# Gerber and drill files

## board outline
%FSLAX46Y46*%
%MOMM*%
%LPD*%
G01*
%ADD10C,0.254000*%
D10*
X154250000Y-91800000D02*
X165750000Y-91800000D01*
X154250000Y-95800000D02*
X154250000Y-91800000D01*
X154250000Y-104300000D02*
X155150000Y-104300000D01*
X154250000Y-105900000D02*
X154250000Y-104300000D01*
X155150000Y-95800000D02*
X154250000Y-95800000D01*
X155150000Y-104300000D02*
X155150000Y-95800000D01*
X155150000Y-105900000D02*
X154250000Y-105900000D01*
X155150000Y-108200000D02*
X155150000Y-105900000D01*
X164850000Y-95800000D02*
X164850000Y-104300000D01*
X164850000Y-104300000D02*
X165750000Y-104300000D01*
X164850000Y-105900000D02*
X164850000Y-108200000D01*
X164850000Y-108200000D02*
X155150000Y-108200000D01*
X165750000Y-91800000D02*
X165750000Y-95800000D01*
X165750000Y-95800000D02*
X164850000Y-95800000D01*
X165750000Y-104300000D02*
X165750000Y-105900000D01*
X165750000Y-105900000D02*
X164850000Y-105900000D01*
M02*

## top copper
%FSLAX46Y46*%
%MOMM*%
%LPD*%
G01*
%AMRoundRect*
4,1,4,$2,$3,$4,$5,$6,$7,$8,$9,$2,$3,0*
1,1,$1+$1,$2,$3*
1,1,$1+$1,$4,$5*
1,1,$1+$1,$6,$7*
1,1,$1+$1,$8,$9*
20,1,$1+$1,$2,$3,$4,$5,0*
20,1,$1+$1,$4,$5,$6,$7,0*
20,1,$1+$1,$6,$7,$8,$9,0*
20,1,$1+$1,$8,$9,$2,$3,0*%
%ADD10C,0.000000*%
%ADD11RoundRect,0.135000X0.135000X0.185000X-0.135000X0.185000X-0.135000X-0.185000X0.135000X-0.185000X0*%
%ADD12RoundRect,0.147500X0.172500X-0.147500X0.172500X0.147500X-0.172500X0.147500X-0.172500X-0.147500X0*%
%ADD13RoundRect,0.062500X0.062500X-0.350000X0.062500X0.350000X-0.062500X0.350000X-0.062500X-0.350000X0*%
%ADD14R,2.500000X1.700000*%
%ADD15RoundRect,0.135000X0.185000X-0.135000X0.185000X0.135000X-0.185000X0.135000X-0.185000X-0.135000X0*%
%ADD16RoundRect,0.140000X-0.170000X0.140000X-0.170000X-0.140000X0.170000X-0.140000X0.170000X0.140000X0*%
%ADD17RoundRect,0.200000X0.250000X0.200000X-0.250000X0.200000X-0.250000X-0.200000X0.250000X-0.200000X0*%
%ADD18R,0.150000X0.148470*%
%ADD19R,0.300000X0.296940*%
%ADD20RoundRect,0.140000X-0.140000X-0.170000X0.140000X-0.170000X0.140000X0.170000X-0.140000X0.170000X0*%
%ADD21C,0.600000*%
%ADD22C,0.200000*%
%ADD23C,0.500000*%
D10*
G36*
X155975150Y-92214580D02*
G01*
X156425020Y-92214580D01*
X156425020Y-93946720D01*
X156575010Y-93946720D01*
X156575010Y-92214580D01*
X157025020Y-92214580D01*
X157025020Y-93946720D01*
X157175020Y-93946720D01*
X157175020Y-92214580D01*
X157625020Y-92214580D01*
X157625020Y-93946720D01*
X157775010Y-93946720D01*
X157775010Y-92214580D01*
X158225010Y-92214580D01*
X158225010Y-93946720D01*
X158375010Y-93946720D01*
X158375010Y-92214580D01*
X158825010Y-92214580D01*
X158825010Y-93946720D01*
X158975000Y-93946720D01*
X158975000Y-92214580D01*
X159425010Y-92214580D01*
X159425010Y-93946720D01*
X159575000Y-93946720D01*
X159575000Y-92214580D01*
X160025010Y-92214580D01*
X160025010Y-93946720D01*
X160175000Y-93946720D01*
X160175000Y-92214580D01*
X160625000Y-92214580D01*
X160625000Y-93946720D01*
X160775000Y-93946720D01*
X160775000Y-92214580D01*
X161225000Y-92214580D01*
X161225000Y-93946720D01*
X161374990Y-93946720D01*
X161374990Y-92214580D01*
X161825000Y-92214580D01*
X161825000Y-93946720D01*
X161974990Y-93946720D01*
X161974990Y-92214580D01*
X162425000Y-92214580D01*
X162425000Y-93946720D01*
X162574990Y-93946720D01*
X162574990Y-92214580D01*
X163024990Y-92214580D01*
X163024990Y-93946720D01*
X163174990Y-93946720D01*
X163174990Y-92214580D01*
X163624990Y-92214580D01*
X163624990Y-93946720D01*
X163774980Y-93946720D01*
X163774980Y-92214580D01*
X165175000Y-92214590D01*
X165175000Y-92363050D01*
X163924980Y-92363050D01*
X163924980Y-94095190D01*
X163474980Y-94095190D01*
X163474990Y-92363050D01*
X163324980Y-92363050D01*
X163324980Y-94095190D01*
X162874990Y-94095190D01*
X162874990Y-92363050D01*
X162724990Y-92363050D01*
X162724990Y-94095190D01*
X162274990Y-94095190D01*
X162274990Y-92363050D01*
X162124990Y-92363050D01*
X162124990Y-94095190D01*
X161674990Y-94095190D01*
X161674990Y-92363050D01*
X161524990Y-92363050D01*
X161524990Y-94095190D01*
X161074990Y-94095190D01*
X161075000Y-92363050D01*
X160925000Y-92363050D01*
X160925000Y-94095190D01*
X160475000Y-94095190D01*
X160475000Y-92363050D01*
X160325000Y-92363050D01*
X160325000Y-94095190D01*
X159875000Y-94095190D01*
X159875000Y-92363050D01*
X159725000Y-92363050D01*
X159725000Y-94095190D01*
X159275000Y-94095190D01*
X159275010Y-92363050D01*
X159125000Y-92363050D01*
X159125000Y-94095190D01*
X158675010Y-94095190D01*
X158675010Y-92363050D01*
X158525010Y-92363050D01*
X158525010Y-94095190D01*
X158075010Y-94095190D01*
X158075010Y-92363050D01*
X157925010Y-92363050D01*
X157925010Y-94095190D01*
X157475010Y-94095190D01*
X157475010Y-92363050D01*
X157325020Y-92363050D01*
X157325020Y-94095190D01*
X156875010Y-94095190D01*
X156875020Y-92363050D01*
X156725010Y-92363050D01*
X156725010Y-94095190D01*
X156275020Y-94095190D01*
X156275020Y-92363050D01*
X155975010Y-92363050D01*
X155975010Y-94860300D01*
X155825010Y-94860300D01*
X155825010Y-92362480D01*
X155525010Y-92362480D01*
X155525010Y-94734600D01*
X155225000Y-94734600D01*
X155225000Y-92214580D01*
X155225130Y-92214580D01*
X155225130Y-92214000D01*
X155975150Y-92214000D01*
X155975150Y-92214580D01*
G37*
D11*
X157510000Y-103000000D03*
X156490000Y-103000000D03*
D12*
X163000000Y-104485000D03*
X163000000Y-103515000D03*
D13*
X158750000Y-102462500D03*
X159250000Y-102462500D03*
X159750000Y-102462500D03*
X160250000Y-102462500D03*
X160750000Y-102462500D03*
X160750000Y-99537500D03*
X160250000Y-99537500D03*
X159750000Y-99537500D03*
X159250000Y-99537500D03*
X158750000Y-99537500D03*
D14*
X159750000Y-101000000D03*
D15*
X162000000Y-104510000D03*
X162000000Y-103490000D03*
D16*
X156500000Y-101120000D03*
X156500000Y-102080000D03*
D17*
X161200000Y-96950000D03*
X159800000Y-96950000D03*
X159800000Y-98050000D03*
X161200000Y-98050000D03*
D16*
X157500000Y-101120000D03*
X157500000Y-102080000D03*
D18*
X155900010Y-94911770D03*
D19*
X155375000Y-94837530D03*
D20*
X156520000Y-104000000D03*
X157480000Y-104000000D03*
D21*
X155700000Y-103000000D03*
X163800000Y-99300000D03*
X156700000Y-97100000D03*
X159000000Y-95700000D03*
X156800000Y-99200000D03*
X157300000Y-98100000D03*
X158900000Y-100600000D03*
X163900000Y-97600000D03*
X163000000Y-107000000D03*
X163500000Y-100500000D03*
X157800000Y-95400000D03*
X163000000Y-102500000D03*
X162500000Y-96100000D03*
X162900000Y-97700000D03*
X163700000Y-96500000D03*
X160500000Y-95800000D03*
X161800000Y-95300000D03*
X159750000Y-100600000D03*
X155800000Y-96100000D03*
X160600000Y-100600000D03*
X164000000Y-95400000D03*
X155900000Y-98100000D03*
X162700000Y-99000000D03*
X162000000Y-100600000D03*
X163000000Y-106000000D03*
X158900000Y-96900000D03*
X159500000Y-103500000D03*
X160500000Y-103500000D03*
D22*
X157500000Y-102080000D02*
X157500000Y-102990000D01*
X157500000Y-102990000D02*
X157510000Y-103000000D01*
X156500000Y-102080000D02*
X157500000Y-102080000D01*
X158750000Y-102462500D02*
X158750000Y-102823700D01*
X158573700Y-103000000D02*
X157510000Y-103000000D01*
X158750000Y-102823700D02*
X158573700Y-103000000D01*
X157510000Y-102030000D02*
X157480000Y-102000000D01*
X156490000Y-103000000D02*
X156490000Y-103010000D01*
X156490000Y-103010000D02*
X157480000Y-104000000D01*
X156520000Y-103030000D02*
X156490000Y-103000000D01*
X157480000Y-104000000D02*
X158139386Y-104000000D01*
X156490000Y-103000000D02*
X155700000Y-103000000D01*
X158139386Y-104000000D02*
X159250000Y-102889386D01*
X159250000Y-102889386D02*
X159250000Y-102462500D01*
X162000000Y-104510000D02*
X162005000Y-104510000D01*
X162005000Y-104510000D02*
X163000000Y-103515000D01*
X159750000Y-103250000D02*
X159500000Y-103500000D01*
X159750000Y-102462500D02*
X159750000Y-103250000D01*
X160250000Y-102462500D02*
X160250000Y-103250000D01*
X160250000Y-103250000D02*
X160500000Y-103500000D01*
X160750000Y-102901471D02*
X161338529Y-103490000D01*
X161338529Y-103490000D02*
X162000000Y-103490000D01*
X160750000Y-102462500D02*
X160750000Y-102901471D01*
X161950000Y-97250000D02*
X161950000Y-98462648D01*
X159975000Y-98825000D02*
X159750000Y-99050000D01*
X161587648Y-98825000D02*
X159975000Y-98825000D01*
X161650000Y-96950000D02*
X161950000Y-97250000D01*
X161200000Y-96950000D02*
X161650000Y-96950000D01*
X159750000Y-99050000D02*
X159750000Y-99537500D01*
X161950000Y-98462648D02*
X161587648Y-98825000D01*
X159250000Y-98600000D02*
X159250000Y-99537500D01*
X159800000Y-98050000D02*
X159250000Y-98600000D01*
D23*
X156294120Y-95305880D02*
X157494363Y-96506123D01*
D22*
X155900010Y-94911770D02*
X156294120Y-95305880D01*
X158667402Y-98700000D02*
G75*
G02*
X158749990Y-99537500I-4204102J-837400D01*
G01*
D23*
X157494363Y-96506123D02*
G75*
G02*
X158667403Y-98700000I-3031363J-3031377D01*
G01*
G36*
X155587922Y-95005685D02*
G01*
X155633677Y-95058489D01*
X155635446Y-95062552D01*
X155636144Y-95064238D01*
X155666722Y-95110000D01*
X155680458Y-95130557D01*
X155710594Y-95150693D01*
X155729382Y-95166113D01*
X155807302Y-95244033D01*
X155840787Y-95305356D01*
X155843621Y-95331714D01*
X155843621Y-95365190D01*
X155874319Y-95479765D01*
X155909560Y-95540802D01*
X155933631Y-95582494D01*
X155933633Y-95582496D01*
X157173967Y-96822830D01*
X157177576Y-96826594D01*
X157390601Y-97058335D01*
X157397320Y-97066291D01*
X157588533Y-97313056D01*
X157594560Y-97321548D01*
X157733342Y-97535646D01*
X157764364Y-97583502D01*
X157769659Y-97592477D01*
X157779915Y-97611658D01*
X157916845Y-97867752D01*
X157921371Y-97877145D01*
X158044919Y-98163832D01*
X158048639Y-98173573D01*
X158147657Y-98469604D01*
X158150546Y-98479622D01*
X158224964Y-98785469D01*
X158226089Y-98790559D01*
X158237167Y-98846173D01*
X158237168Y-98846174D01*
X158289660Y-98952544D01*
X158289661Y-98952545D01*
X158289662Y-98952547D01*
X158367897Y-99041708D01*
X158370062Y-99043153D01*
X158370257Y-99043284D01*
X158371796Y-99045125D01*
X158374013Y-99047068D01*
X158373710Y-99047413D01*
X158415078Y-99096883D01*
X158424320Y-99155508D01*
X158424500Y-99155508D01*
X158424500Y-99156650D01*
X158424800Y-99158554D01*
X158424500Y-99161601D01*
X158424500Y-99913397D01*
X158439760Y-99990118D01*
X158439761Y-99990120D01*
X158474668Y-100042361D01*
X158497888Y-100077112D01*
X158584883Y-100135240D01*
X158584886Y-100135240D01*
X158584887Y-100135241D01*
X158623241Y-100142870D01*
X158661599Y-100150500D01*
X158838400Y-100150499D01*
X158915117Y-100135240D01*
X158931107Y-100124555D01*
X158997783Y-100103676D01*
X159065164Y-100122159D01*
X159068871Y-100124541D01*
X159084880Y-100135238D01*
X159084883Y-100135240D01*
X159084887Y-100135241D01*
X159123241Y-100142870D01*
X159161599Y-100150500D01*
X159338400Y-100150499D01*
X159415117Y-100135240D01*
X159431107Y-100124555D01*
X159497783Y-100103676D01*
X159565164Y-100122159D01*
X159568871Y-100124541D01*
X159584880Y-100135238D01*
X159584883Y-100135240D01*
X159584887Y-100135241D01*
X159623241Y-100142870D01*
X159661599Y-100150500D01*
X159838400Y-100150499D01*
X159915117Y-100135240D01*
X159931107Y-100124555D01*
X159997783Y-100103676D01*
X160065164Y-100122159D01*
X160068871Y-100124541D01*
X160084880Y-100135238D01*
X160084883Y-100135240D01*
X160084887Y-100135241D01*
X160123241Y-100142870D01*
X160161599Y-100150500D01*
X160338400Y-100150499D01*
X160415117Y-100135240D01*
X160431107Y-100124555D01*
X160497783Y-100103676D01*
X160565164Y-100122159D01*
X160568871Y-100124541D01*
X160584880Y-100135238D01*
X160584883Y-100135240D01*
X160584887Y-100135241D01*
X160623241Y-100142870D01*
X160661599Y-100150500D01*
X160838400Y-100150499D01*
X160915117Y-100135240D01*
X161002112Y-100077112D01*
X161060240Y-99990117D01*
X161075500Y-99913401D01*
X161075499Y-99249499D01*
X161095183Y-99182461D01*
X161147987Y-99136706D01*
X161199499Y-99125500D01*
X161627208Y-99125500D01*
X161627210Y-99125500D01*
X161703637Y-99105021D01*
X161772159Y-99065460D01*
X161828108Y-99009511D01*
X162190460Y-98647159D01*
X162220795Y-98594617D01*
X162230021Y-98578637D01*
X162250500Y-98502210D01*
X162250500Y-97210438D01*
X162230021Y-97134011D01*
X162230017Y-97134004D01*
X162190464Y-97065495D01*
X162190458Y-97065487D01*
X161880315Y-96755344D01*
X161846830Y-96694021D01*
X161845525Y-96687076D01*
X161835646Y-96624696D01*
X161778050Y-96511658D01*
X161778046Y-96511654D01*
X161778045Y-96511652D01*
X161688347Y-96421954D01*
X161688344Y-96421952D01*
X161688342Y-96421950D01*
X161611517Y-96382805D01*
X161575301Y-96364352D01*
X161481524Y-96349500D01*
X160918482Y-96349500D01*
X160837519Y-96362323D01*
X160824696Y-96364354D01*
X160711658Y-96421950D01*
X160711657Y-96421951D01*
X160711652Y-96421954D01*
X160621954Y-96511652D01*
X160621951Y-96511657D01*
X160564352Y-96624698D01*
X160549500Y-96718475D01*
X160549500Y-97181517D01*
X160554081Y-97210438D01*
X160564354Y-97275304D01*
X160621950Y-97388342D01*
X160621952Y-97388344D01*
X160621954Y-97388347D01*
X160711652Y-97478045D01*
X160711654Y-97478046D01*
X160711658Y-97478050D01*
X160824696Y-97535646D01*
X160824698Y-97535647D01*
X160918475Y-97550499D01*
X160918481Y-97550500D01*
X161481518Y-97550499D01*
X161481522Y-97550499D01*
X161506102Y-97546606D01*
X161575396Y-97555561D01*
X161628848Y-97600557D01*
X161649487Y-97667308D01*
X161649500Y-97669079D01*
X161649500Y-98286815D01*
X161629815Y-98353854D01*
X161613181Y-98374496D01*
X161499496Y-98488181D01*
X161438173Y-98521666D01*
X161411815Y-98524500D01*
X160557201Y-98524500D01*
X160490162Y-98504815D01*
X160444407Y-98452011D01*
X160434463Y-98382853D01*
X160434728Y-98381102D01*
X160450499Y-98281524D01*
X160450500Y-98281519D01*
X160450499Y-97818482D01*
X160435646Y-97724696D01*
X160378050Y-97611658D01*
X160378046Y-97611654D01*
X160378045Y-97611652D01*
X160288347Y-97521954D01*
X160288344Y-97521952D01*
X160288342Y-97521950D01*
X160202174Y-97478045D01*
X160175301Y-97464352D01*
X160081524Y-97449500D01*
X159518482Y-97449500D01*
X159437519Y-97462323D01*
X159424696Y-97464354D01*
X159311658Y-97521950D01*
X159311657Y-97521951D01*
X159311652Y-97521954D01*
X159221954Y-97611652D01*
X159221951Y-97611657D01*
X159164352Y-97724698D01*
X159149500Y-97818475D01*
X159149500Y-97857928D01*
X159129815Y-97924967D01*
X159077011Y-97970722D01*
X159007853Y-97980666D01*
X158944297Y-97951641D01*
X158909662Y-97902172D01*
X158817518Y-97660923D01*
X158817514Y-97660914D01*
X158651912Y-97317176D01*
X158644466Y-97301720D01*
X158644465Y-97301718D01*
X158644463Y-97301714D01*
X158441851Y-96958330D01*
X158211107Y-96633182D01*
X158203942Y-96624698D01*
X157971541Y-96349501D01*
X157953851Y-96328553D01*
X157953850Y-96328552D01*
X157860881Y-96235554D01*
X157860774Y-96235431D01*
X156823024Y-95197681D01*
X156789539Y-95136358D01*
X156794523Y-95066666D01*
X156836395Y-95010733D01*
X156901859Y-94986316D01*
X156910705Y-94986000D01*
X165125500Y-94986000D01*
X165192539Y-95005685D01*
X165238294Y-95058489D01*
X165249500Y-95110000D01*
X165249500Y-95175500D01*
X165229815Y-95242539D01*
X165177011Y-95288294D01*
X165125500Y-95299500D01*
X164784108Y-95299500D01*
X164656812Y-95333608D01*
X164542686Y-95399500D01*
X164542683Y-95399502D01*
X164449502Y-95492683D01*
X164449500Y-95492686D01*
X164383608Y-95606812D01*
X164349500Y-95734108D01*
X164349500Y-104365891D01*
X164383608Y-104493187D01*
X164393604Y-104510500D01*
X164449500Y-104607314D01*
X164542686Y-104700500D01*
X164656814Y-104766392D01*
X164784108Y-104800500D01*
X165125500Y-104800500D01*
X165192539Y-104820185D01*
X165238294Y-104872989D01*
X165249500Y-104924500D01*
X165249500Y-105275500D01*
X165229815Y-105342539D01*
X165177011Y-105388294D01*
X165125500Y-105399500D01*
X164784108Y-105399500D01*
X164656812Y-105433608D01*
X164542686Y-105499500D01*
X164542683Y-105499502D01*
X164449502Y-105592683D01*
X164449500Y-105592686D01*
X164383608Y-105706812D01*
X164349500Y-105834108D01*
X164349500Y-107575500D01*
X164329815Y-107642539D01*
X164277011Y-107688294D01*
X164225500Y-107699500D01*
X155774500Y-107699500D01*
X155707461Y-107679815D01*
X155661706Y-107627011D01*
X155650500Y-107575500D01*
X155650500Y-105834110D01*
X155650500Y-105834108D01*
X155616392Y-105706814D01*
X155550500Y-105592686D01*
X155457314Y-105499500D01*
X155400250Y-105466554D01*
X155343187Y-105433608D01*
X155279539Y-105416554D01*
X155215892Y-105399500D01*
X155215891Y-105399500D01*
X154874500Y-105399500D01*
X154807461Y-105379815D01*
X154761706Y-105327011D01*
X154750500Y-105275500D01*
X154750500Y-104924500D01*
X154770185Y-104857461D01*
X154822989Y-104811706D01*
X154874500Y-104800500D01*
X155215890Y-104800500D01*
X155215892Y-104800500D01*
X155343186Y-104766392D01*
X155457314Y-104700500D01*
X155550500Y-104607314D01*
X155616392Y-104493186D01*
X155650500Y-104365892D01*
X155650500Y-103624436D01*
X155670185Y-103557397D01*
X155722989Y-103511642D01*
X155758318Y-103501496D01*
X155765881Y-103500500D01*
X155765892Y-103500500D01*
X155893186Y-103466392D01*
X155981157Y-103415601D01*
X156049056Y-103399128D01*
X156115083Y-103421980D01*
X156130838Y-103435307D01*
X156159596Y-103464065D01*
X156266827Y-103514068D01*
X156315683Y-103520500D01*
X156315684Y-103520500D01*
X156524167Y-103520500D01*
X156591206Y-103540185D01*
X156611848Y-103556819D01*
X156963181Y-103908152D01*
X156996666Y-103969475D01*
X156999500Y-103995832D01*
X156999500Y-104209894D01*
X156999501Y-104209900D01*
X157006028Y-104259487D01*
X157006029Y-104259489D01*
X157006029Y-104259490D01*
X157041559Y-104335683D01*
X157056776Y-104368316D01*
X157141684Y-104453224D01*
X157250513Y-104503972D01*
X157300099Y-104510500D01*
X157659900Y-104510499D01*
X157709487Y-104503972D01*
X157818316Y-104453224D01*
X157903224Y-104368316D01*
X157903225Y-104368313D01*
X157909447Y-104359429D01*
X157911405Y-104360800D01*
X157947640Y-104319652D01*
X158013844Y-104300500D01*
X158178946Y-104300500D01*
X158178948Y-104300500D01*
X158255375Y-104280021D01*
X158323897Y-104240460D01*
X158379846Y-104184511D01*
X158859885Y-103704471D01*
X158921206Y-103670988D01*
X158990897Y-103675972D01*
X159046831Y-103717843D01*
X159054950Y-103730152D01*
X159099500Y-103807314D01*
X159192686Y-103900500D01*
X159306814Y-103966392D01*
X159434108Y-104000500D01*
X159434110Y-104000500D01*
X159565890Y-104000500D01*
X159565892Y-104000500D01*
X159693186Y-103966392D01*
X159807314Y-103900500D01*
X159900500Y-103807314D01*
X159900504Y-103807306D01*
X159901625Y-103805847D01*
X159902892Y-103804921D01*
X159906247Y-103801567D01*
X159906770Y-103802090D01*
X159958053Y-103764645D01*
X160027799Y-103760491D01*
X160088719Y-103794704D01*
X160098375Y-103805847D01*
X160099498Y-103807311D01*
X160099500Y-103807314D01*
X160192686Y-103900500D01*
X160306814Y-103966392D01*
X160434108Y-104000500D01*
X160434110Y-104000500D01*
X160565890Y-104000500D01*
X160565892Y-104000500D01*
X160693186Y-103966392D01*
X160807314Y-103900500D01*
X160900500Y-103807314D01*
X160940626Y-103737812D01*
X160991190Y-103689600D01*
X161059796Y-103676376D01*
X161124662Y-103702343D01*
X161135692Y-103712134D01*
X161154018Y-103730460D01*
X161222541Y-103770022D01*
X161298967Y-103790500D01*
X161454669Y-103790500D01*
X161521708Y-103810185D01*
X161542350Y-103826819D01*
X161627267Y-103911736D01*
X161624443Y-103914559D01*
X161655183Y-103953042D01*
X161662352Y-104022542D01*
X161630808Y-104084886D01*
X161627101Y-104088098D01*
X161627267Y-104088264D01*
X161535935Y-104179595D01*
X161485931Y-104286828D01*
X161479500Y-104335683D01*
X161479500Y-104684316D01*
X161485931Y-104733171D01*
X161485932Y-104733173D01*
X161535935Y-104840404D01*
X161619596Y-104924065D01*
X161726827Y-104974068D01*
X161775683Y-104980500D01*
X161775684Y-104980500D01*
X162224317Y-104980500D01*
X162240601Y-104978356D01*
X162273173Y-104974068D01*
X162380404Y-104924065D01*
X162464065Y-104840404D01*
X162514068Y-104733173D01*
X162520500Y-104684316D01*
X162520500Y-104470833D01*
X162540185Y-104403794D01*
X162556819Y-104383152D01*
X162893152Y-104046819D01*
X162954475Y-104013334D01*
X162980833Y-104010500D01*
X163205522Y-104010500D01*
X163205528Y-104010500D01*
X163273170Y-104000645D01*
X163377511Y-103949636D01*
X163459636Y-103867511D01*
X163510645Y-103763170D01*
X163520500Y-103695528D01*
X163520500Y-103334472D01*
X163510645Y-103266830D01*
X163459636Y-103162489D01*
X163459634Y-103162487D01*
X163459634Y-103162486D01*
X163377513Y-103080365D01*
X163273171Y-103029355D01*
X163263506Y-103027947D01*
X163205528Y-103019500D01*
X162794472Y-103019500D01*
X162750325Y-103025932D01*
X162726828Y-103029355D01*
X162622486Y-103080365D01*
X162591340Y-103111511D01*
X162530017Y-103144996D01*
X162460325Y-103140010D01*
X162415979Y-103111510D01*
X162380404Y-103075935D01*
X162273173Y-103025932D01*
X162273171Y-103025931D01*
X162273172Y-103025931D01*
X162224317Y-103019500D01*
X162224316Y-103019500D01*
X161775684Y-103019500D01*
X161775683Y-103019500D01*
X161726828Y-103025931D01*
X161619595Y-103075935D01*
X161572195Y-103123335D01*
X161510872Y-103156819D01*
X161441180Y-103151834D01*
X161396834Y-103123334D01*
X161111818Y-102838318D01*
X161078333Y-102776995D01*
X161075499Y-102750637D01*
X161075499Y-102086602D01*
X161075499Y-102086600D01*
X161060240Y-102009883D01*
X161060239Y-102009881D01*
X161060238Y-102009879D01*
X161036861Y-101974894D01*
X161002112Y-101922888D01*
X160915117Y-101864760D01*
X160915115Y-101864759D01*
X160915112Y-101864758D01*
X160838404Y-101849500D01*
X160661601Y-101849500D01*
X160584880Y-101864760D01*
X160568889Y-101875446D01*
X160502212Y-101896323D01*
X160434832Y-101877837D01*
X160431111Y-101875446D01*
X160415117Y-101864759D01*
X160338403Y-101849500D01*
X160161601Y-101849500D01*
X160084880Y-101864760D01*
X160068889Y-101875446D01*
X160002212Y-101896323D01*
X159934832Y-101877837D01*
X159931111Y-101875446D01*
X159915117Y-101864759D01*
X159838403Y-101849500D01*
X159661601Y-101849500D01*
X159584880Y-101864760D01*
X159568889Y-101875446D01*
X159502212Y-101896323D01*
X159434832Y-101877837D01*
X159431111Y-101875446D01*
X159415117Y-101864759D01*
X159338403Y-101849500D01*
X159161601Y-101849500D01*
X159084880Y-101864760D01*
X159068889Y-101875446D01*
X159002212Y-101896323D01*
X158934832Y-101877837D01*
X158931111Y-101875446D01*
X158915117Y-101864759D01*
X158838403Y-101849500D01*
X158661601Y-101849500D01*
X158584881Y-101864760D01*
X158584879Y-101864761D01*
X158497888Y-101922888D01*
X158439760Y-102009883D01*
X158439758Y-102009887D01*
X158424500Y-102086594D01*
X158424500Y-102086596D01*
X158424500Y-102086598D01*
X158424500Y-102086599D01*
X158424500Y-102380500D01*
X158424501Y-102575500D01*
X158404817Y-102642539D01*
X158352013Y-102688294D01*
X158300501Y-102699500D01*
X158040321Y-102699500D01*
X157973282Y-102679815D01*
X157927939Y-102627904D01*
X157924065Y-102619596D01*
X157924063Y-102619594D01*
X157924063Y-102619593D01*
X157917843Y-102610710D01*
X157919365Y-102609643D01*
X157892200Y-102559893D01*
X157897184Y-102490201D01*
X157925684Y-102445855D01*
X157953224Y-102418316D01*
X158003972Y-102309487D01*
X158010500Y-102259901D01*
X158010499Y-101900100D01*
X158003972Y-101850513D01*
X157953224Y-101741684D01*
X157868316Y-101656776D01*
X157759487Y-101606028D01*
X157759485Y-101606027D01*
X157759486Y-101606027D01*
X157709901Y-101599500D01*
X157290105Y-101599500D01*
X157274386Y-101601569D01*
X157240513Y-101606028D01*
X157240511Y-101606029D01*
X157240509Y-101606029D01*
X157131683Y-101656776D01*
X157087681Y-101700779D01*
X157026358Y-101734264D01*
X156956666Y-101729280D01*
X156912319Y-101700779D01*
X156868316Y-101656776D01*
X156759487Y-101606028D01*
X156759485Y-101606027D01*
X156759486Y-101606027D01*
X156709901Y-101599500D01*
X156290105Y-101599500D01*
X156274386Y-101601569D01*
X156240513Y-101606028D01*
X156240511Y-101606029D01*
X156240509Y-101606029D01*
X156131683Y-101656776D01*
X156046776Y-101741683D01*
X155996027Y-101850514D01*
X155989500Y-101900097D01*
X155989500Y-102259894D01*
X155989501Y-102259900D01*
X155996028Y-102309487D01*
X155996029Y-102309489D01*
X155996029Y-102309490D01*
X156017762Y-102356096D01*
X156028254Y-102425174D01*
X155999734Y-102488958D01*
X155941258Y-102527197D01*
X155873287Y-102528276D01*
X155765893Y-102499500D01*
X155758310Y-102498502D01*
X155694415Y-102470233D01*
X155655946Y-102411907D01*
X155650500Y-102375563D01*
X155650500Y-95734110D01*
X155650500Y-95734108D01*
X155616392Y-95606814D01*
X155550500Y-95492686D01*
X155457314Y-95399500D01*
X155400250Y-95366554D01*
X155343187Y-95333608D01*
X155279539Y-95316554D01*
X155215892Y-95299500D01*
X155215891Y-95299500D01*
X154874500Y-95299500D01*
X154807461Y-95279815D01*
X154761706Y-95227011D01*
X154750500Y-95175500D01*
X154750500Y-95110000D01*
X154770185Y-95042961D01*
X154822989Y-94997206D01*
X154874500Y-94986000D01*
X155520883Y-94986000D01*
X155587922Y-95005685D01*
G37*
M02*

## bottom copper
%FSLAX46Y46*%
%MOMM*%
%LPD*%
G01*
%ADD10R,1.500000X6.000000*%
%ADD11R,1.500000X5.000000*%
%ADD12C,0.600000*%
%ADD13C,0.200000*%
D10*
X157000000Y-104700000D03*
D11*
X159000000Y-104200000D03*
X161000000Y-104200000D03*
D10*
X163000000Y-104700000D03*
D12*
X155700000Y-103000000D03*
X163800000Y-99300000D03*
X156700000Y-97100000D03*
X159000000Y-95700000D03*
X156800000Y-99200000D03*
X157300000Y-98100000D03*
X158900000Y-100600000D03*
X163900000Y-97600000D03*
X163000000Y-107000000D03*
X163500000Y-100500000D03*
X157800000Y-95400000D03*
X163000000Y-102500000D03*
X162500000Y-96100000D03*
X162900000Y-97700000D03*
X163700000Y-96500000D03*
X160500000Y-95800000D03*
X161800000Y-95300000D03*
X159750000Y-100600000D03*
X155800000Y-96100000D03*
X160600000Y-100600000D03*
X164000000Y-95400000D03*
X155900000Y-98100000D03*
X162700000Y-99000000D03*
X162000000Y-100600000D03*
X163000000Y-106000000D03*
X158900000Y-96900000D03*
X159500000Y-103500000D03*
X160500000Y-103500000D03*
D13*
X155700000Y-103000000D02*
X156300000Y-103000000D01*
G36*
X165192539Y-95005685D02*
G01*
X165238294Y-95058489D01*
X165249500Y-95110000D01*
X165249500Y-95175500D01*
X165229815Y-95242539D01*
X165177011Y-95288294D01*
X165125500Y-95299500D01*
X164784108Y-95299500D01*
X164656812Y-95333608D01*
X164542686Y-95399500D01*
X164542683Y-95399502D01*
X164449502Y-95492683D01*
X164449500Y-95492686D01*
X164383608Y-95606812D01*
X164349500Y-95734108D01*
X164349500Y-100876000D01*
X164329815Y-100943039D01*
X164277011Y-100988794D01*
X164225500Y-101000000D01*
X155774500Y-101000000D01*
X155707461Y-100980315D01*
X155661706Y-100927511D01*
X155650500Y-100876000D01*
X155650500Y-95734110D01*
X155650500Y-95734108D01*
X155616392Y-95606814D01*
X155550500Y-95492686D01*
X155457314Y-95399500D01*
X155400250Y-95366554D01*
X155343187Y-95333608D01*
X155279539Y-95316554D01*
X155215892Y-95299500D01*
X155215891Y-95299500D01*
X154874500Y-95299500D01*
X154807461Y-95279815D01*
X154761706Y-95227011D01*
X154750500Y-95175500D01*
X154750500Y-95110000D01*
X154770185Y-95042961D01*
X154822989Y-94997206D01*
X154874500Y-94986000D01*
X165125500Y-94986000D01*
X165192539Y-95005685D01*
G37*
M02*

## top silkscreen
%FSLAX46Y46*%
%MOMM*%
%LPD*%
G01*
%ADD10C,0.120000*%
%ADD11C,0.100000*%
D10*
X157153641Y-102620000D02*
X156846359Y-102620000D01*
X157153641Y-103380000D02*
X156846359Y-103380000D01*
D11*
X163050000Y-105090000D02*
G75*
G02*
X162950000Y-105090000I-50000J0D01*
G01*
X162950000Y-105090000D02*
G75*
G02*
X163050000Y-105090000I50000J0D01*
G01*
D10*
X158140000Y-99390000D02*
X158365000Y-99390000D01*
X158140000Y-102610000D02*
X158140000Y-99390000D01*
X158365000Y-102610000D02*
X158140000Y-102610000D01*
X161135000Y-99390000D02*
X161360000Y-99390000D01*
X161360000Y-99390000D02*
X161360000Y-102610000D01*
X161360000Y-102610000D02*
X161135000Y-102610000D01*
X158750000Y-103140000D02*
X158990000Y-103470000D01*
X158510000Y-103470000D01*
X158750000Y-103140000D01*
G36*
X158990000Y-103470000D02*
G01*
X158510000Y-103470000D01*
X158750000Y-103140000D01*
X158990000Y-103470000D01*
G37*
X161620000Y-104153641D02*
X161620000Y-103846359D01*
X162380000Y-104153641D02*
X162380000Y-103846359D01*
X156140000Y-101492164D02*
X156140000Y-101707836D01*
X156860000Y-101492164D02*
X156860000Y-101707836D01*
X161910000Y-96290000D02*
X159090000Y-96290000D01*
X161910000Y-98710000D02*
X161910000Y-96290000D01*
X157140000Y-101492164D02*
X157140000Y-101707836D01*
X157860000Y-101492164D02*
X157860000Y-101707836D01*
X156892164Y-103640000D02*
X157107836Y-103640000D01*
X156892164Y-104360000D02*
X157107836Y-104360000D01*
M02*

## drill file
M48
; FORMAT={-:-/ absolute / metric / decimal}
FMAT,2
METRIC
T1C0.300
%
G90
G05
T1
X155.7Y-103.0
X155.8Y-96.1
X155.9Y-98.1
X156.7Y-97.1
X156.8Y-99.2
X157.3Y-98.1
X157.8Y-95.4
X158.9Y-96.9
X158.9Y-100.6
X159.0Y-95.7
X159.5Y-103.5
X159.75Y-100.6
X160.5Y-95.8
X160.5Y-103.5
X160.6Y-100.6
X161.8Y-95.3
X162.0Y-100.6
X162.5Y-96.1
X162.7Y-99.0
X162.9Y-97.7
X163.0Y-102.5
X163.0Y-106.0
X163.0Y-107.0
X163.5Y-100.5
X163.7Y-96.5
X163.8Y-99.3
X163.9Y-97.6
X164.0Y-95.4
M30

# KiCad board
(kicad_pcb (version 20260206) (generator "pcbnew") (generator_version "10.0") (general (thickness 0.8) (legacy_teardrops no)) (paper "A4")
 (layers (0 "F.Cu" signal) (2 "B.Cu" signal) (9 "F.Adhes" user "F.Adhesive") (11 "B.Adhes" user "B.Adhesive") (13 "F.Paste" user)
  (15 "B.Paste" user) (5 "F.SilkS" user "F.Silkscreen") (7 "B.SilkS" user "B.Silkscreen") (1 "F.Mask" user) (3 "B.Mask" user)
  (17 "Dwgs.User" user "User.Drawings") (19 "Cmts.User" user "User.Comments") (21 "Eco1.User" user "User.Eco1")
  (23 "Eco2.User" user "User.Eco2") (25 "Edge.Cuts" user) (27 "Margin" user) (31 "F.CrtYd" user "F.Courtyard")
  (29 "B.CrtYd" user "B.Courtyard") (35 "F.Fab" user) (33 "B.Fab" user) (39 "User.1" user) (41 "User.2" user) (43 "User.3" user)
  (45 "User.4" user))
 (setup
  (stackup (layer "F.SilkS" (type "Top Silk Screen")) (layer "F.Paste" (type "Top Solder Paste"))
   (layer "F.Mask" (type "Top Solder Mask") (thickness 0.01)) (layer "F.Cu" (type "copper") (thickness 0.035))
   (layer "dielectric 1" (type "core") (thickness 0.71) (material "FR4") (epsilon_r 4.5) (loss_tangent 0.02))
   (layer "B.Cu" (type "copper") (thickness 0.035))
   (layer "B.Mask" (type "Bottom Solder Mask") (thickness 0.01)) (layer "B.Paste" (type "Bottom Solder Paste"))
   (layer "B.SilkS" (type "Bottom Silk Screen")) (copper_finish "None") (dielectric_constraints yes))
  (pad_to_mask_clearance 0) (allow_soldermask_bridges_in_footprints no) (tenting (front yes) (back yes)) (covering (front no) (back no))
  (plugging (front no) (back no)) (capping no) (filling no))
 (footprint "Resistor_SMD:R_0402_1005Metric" (layer "F.Cu") (at 157 103 180)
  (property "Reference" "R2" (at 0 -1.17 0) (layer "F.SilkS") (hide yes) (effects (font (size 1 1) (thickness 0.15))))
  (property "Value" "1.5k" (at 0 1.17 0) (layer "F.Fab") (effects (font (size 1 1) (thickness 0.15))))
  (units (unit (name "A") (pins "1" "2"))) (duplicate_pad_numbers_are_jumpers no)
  (fp_line (start -0.153641 0.38) (end 0.153641 0.38) (stroke (width 0.12) (type solid)) (layer "F.SilkS"))
  (fp_line (start -0.153641 -0.38) (end 0.153641 -0.38) (stroke (width 0.12) (type solid)) (layer "F.SilkS"))
  (pad "1" smd roundrect (at -0.51 0 180) (size 0.54 0.64) (layers "F.Cu" "F.Mask" "F.Paste") (roundrect_rratio 0.25) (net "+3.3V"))
  (pad "2" smd roundrect (at 0.51 0 180) (size 0.54 0.64) (layers "F.Cu" "F.Mask" "F.Paste") (roundrect_rratio 0.25) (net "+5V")))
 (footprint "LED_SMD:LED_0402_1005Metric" (layer "F.Cu") (at 163 104 90)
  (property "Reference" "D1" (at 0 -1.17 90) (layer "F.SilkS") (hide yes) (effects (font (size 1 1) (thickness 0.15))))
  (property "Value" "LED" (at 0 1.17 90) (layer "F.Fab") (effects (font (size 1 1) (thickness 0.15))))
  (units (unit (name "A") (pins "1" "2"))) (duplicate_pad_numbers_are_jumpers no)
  (fp_circle (center -1.09 0) (end -1.04 0) (stroke (width 0.1) (type solid)) (fill no) (layer "F.SilkS"))
  (pad "1" smd roundrect (at -0.485 0 90) (size 0.59 0.64) (layers "F.Cu" "F.Mask" "F.Paste") (roundrect_rratio 0.25) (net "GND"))
  (pad "2" smd roundrect (at 0.485 0 90) (size 0.59 0.64) (layers "F.Cu" "F.Mask" "F.Paste") (roundrect_rratio 0.25) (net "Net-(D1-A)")))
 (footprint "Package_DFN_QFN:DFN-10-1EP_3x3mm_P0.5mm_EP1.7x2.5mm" (layer "F.Cu") (at 159.75 101 90)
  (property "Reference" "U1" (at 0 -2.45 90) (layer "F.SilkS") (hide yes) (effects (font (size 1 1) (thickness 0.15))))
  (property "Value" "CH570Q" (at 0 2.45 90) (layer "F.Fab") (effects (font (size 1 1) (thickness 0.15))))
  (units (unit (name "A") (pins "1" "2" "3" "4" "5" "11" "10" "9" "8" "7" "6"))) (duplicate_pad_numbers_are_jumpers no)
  (fp_line (start 1.61 -1.61) (end 1.61 -1.385) (stroke (width 0.12) (type solid)) (layer "F.SilkS"))
  (fp_line (start -1.61 -1.61) (end 1.61 -1.61) (stroke (width 0.12) (type solid)) (layer "F.SilkS"))
  (fp_line (start -1.61 -1.385) (end -1.61 -1.61) (stroke (width 0.12) (type solid)) (layer "F.SilkS"))
  (fp_line (start 1.61 1.385) (end 1.61 1.61) (stroke (width 0.12) (type solid)) (layer "F.SilkS"))
  (fp_line (start 1.61 1.61) (end -1.61 1.61) (stroke (width 0.12) (type solid)) (layer "F.SilkS"))
  (fp_line (start -1.61 1.61) (end -1.61 1.385) (stroke (width 0.12) (type solid)) (layer "F.SilkS"))
  (fp_poly (pts (xy -2.14 -1) (xy -2.47 -0.76) (xy -2.47 -1.24)) (stroke (width 0.12) (type solid)) (fill yes) (layer "F.SilkS"))
  (pad "" smd roundrect (at -0.425 -0.625 90) (size 0.69 1.01) (layers "F.Paste") (roundrect_rratio 0.25))
  (pad "" smd roundrect (at -0.425 0.625 90) (size 0.69 1.01) (layers "F.Paste") (roundrect_rratio 0.25))
  (pad "" smd roundrect (at 0.425 -0.625 90) (size 0.69 1.01) (layers "F.Paste") (roundrect_rratio 0.25))
  (pad "" smd roundrect (at 0.425 0.625 90) (size 0.69 1.01) (layers "F.Paste") (roundrect_rratio 0.25))
  (pad "1" smd roundrect (at -1.4625 -1 90) (size 0.825 0.25) (layers "F.Cu" "F.Mask" "F.Paste") (roundrect_rratio 0.25) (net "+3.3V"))
  (pad "2" smd roundrect (at -1.4625 -0.5 90) (size 0.825 0.25) (layers "F.Cu" "F.Mask" "F.Paste") (roundrect_rratio 0.25) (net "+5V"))
  (pad "3" smd roundrect (at -1.4625 0 90) (size 0.825 0.25) (layers "F.Cu" "F.Mask" "F.Paste") (roundrect_rratio 0.25) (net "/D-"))
  (pad "4" smd roundrect (at -1.4625 0.5 90) (size 0.825 0.25) (layers "F.Cu" "F.Mask" "F.Paste") (roundrect_rratio 0.25) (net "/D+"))
  (pad "5" smd roundrect (at -1.4625 1 90) (size 0.825 0.25) (layers "F.Cu" "F.Mask" "F.Paste") (roundrect_rratio 0.25) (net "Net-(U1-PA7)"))
  (pad "6" smd roundrect (at 1.4625 1 90) (size 0.825 0.25) (layers "F.Cu" "F.Mask" "F.Paste") (roundrect_rratio 0.25)
   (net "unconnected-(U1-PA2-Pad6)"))
  (pad "7" smd roundrect (at 1.4625 0.5 90) (size 0.825 0.25) (layers "F.Cu" "F.Mask" "F.Paste") (roundrect_rratio 0.25)
   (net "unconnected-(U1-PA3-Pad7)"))
  (pad "8" smd roundrect (at 1.4625 0 90) (size 0.825 0.25) (layers "F.Cu" "F.Mask" "F.Paste") (roundrect_rratio 0.25) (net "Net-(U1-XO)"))
  (pad "9" smd roundrect (at 1.4625 -0.5 90) (size 0.825 0.25) (layers "F.Cu" "F.Mask" "F.Paste") (roundrect_rratio 0.25)
   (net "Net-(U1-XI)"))
  (pad "10" smd roundrect (at 1.4625 -1 90) (size 0.825 0.25) (layers "F.Cu" "F.Mask" "F.Paste") (roundrect_rratio 0.25)
   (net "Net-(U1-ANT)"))
  (pad "11" smd rect (at 0 0 90) (size 1.7 2.5) (layers "F.Cu" "F.Mask") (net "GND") (zone_connect 2)))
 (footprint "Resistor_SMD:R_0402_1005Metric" (layer "F.Cu") (at 162 104 90)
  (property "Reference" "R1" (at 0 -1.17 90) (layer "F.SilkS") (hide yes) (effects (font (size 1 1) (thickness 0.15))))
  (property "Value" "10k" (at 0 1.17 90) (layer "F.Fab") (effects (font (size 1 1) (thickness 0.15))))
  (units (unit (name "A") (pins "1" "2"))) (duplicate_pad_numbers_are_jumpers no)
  (fp_line (start -0.153641 -0.38) (end 0.153641 -0.38) (stroke (width 0.12) (type solid)) (layer "F.SilkS"))
  (fp_line (start -0.153641 0.38) (end 0.153641 0.38) (stroke (width 0.12) (type solid)) (layer "F.SilkS"))
  (pad "1" smd roundrect (at -0.51 0 90) (size 0.54 0.64) (layers "F.Cu" "F.Mask" "F.Paste") (roundrect_rratio 0.25) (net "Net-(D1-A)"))
  (pad "2" smd roundrect (at 0.51 0 90) (size 0.54 0.64) (layers "F.Cu" "F.Mask" "F.Paste") (roundrect_rratio 0.25) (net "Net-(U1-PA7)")))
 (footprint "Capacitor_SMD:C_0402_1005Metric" (layer "F.Cu") (at 156.5 101.6 -90)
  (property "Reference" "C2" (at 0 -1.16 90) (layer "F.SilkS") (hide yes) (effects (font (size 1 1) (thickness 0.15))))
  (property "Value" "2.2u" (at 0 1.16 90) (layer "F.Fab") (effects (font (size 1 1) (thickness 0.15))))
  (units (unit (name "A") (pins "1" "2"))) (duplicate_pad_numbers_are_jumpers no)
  (fp_line (start -0.107836 0.36) (end 0.107836 0.36) (stroke (width 0.12) (type solid)) (layer "F.SilkS"))
  (fp_line (start -0.107836 -0.36) (end 0.107836 -0.36) (stroke (width 0.12) (type solid)) (layer "F.SilkS"))
  (pad "1" smd roundrect (at -0.48 0 270) (size 0.56 0.62) (layers "F.Cu" "F.Mask" "F.Paste") (roundrect_rratio 0.25) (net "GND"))
  (pad "2" smd roundrect (at 0.48 0 270) (size 0.56 0.62) (layers "F.Cu" "F.Mask" "F.Paste") (roundrect_rratio 0.25) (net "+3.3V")))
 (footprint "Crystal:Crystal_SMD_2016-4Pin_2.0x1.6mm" (layer "F.Cu") (at 160.5 97.5 180)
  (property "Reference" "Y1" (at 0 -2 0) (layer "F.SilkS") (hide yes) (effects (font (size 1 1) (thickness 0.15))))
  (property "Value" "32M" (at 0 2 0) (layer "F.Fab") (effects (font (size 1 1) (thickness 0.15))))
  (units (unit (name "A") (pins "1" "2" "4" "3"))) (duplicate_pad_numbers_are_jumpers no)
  (fp_line (start -1.41 1.21) (end 1.41 1.21) (stroke (width 0.12) (type solid)) (layer "F.SilkS"))
  (fp_line (start -1.41 -1.21) (end -1.41 1.21) (stroke (width 0.12) (type solid)) (layer "F.SilkS"))
  (pad "1" smd roundrect (at -0.7 0.55 180) (size 0.9 0.8) (layers "F.Cu" "F.Mask" "F.Paste") (roundrect_rratio 0.25) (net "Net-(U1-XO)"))
  (pad "2" smd roundrect (at 0.7 0.55 180) (size 0.9 0.8) (layers "F.Cu" "F.Mask" "F.Paste") (roundrect_rratio 0.25) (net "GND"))
  (pad "3" smd roundrect (at 0.7 -0.55 180) (size 0.9 0.8) (layers "F.Cu" "F.Mask" "F.Paste") (roundrect_rratio 0.25) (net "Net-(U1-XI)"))
  (pad "4" smd roundrect (at -0.7 -0.55 180) (size 0.9 0.8) (layers "F.Cu" "F.Mask" "F.Paste") (roundrect_rratio 0.25) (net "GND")))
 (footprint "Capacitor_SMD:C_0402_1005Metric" (layer "F.Cu") (at 157.5 101.6 -90)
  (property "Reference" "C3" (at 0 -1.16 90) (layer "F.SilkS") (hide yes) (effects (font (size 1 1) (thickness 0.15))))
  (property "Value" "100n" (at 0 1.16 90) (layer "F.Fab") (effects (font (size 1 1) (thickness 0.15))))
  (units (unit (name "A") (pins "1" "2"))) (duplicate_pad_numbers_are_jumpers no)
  (fp_line (start -0.107836 0.36) (end 0.107836 0.36) (stroke (width 0.12) (type solid)) (layer "F.SilkS"))
  (fp_line (start -0.107836 -0.36) (end 0.107836 -0.36) (stroke (width 0.12) (type solid)) (layer "F.SilkS"))
  (pad "1" smd roundrect (at -0.48 0 270) (size 0.56 0.62) (layers "F.Cu" "F.Mask" "F.Paste") (roundrect_rratio 0.25) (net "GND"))
  (pad "2" smd roundrect (at 0.48 0 270) (size 0.56 0.62) (layers "F.Cu" "F.Mask" "F.Paste") (roundrect_rratio 0.25) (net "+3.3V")))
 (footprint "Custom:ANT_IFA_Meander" (layer "F.Cu") (at 155.90001 94.91177)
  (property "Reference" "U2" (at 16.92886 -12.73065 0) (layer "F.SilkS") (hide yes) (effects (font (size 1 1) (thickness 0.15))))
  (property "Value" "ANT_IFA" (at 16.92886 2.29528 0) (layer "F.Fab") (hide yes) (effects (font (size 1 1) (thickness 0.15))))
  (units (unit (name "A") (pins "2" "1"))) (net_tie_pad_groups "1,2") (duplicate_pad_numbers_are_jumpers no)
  (fp_poly
   (pts (xy -0.67501 -0.17717) (xy -0.375 -0.17717) (xy -0.375 -2.54929) (xy -0.075 -2.54929) (xy -0.075 -0.05147) (xy 0.075 -0.05147)
    (xy 0.075 -2.54872) (xy 0.37501 -2.54872) (xy 0.37501 -0.81658) (xy 0.825 -0.81658) (xy 0.825 -2.54872) (xy 0.97501 -2.54872)
    (xy 0.975 -0.81658) (xy 1.42501 -0.81658) (xy 1.42501 -2.54872) (xy 1.575 -2.54872) (xy 1.575 -0.81658) (xy 2.025 -0.81658)
    (xy 2.025 -2.54872) (xy 2.175 -2.54872) (xy 2.175 -0.81658) (xy 2.625 -0.81658) (xy 2.625 -2.54872) (xy 2.775 -2.54872)
    (xy 2.775 -0.81658) (xy 3.22499 -0.81658) (xy 3.22499 -2.54872) (xy 3.375 -2.54872) (xy 3.37499 -0.81658) (xy 3.82499 -0.81658)
    (xy 3.82499 -2.54872) (xy 3.97499 -2.54872) (xy 3.97499 -0.81658) (xy 4.42499 -0.81658) (xy 4.42499 -2.54872) (xy 4.57499 -2.54872)
    (xy 4.57499 -0.81658) (xy 5.02499 -0.81658) (xy 5.02499 -2.54872) (xy 5.17499 -2.54872) (xy 5.17498 -0.81658) (xy 5.62498 -0.81658)
    (xy 5.62498 -2.54872) (xy 5.77498 -2.54872) (xy 5.77498 -0.81658) (xy 6.22498 -0.81658) (xy 6.22498 -2.54872) (xy 6.37498 -2.54872)
    (xy 6.37498 -0.81658) (xy 6.82498 -0.81658) (xy 6.82498 -2.54872) (xy 6.97498 -2.54872) (xy 6.97498 -0.81658) (xy 7.42497 -0.81658)
    (xy 7.42497 -2.54872) (xy 7.57498 -2.54872) (xy 7.57497 -0.81658) (xy 8.02497 -0.81658) (xy 8.02497 -2.54872) (xy 9.27499 -2.54872)
    (xy 9.27499 -2.69718) (xy 7.87497 -2.69719) (xy 7.87497 -0.96505) (xy 7.72498 -0.96505) (xy 7.72498 -2.69719) (xy 7.27498 -2.69719)
    (xy 7.27498 -0.96505) (xy 7.12498 -0.96505) (xy 7.12498 -2.69719) (xy 6.67498 -2.69719) (xy 6.67498 -0.96505) (xy 6.52499 -0.96505)
    (xy 6.52499 -2.69719) (xy 6.07498 -2.69719) (xy 6.07498 -0.96505) (xy 5.92499 -0.96505) (xy 5.92499 -2.69719) (xy 5.47498 -2.69719)
    (xy 5.47498 -0.96505) (xy 5.32499 -0.96505) (xy 5.32499 -2.69719) (xy 4.87499 -2.69719) (xy 4.87499 -0.96505) (xy 4.72499 -0.96505)
    (xy 4.72499 -2.69719) (xy 4.27499 -2.69719) (xy 4.27499 -0.96505) (xy 4.125 -0.96505) (xy 4.125 -2.69719) (xy 3.67499 -2.69719)
    (xy 3.67499 -0.96505) (xy 3.525 -0.96505) (xy 3.525 -2.69719) (xy 3.07499 -2.69719) (xy 3.07499 -0.96505) (xy 2.925 -0.96505)
    (xy 2.925 -2.69719) (xy 2.475 -2.69719) (xy 2.475 -0.96505) (xy 2.325 -0.96505) (xy 2.325 -2.69719) (xy 1.875 -2.69719)
    (xy 1.875 -0.96505) (xy 1.72501 -0.96505) (xy 1.72501 -2.69719) (xy 1.27501 -2.69719) (xy 1.27501 -0.96505) (xy 1.12501 -0.96505)
    (xy 1.12501 -2.69719) (xy 0.675 -2.69719) (xy 0.675 -0.96505) (xy 0.52501 -0.96505) (xy 0.52501 -2.69719) (xy 0.07514 -2.69719)
    (xy 0.07514 -2.69777) (xy -0.67488 -2.69777) (xy -0.67488 -2.69719) (xy -0.67501 -2.69719) (xy -0.67501 -0.17717))
   (stroke (width 0) (type solid)) (fill yes) (layer "F.Cu"))
  (pad "1" smd rect (at 0 0) (size 0.15 0.14847) (layers "F.Cu" "F.Mask") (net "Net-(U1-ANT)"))
  (pad "2" smd rect (at -0.52501 -0.07424) (size 0.3 0.29694) (layers "F.Cu" "F.Mask") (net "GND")))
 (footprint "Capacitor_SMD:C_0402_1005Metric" (layer "F.Cu") (at 157 104)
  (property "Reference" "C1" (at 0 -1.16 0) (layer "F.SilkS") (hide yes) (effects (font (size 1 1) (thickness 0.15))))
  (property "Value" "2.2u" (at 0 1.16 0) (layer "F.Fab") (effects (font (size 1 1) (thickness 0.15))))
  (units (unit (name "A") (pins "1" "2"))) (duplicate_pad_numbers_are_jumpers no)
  (fp_line (start -0.107836 -0.36) (end 0.107836 -0.36) (stroke (width 0.12) (type solid)) (layer "F.SilkS"))
  (fp_line (start -0.107836 0.36) (end 0.107836 0.36) (stroke (width 0.12) (type solid)) (layer "F.SilkS"))
  (pad "1" smd roundrect (at -0.48 0) (size 0.56 0.62) (layers "F.Cu" "F.Mask" "F.Paste") (roundrect_rratio 0.25) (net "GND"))
  (pad "2" smd roundrect (at 0.48 0) (size 0.56 0.62) (layers "F.Cu" "F.Mask" "F.Paste") (roundrect_rratio 0.25) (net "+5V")))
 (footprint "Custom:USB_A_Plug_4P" (layer "B.Cu") (at 160 108.2 180)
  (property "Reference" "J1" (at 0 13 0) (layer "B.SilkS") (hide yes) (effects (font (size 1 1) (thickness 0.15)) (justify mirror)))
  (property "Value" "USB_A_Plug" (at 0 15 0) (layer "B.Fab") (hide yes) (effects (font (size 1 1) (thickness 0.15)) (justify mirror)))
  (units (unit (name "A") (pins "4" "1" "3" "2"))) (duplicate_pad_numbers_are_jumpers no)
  (pad "1" smd rect (at 3 3.5 180) (size 1.5 6) (layers "B.Cu" "B.Mask") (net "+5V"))
  (pad "2" smd rect (at 1 4 180) (size 1.5 5) (layers "B.Cu" "B.Mask") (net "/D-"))
  (pad "3" smd rect (at -1 4 180) (size 1.5 5) (layers "B.Cu" "B.Mask") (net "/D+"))
  (pad "4" smd rect (at -3 3.5 180) (size 1.5 6) (layers "B.Cu" "B.Mask") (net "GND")))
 (gr_line (start 154.25 91.8) (end 165.75 91.8) (stroke (width 0.254) (type solid)) (layer "Edge.Cuts"))
 (gr_line (start 154.25 95.8) (end 154.25 91.8) (stroke (width 0.254) (type solid)) (layer "Edge.Cuts"))
 (gr_line (start 154.25 104.3) (end 155.15 104.3) (stroke (width 0.254) (type solid)) (layer "Edge.Cuts"))
 (gr_line (start 154.25 105.9) (end 154.25 104.3) (stroke (width 0.254) (type solid)) (layer "Edge.Cuts"))
 (gr_line (start 155.15 95.8) (end 154.25 95.8) (stroke (width 0.254) (type solid)) (layer "Edge.Cuts"))
 (gr_line (start 155.15 104.3) (end 155.15 95.8) (stroke (width 0.254) (type solid)) (layer "Edge.Cuts"))
 (gr_line (start 155.15 105.9) (end 154.25 105.9) (stroke (width 0.254) (type solid)) (layer "Edge.Cuts"))
 (gr_line (start 155.15 108.2) (end 155.15 105.9) (stroke (width 0.254) (type solid)) (layer "Edge.Cuts"))
 (gr_line (start 164.85 95.8) (end 164.85 104.3) (stroke (width 0.254) (type solid)) (layer "Edge.Cuts"))
 (gr_line (start 164.85 104.3) (end 165.75 104.3) (stroke (width 0.254) (type solid)) (layer "Edge.Cuts"))
 (gr_line (start 164.85 105.9) (end 164.85 108.2) (stroke (width 0.254) (type solid)) (layer "Edge.Cuts"))
 (gr_line (start 164.85 108.2) (end 155.15 108.2) (stroke (width 0.254) (type solid)) (layer "Edge.Cuts"))
 (gr_line (start 165.75 91.8) (end 165.75 95.8) (stroke (width 0.254) (type solid)) (layer "Edge.Cuts"))
 (gr_line (start 165.75 95.8) (end 164.85 95.8) (stroke (width 0.254) (type solid)) (layer "Edge.Cuts"))
 (gr_line (start 165.75 104.3) (end 165.75 105.9) (stroke (width 0.254) (type solid)) (layer "Edge.Cuts"))
 (gr_line (start 165.75 105.9) (end 164.85 105.9) (stroke (width 0.254) (type solid)) (layer "Edge.Cuts"))
 (segment (start 157.5 102.08) (end 157.5 102.99) (width 0.2) (layer "F.Cu") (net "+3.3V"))
 (segment (start 157.5 102.99) (end 157.51 103) (width 0.2) (layer "F.Cu") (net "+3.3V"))
 (segment (start 156.5 102.08) (end 157.5 102.08) (width 0.2) (layer "F.Cu") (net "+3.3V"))
 (segment (start 158.75 102.4625) (end 158.75 102.8237) (width 0.2) (layer "F.Cu") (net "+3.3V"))
 (segment (start 158.5737 103) (end 157.51 103) (width 0.2) (layer "F.Cu") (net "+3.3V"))
 (segment (start 158.75 102.8237) (end 158.5737 103) (width 0.2) (layer "F.Cu") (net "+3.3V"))
 (segment (start 157.51 102.03) (end 157.48 102) (width 0.2) (layer "F.Cu") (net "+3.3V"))
 (segment (start 156.49 103) (end 156.49 103.01) (width 0.2) (layer "F.Cu") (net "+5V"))
 (segment (start 156.49 103.01) (end 157.48 104) (width 0.2) (layer "F.Cu") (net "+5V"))
 (segment (start 156.52 103.03) (end 156.49 103) (width 0.2) (layer "F.Cu") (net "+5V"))
 (segment (start 157.48 104) (end 158.139386 104) (width 0.2) (layer "F.Cu") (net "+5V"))
 (segment (start 156.49 103) (end 155.7 103) (width 0.2) (layer "F.Cu") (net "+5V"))
 (segment (start 158.139386 104) (end 159.25 102.889386) (width 0.2) (layer "F.Cu") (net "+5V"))
 (segment (start 159.25 102.889386) (end 159.25 102.4625) (width 0.2) (layer "F.Cu") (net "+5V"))
 (via (at 155.7 103) (size 0.6) (drill 0.3) (layers "F.Cu" "B.Cu") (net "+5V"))
 (segment (start 155.7 103) (end 156.3 103) (width 0.2) (layer "B.Cu") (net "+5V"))
 (via (at 163.8 99.3) (size 0.6) (drill 0.3) (layers "F.Cu" "B.Cu") (free yes) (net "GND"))
 (via (at 156.7 97.1) (size 0.6) (drill 0.3) (layers "F.Cu" "B.Cu") (free yes) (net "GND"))
 (via (at 159 95.7) (size 0.6) (drill 0.3) (layers "F.Cu" "B.Cu") (free yes) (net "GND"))
 (via (at 156.8 99.2) (size 0.6) (drill 0.3) (layers "F.Cu" "B.Cu") (free yes) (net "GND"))
 (via (at 157.3 98.1) (size 0.6) (drill 0.3) (layers "F.Cu" "B.Cu") (free yes) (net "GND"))
 (via (at 158.9 100.6) (size 0.6) (drill 0.3) (layers "F.Cu" "B.Cu") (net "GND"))
 (via (at 163.9 97.6) (size 0.6) (drill 0.3) (layers "F.Cu" "B.Cu") (free yes) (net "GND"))
 (via (at 163 107) (size 0.6) (drill 0.3) (layers "F.Cu" "B.Cu") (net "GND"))
 (via (at 163.5 100.5) (size 0.6) (drill 0.3) (layers "F.Cu" "B.Cu") (free yes) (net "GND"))
 (via (at 157.8 95.4) (size 0.6) (drill 0.3) (layers "F.Cu" "B.Cu") (free yes) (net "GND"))
 (via (at 163 102.5) (size 0.6) (drill 0.3) (layers "F.Cu" "B.Cu") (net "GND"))
 (via (at 162.5 96.1) (size 0.6) (drill 0.3) (layers "F.Cu" "B.Cu") (free yes) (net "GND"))
 (via (at 162.9 97.7) (size 0.6) (drill 0.3) (layers "F.Cu" "B.Cu") (free yes) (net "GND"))
 (via (at 163.7 96.5) (size 0.6) (drill 0.3) (layers "F.Cu" "B.Cu") (free yes) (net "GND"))
 (via (at 160.5 95.8) (size 0.6) (drill 0.3) (layers "F.Cu" "B.Cu") (free yes) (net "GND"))
 (via (at 161.8 95.3) (size 0.6) (drill 0.3) (layers "F.Cu" "B.Cu") (free yes) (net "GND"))
 (via (at 159.75 100.6) (size 0.6) (drill 0.3) (layers "F.Cu" "B.Cu") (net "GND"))
 (via (at 155.8 96.1) (size 0.6) (drill 0.3) (layers "F.Cu" "B.Cu") (free yes) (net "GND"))
 (via (at 160.6 100.6) (size 0.6) (drill 0.3) (layers "F.Cu" "B.Cu") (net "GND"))
 (via (at 164 95.4) (size 0.6) (drill 0.3) (layers "F.Cu" "B.Cu") (free yes) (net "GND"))
 (via (at 155.9 98.1) (size 0.6) (drill 0.3) (layers "F.Cu" "B.Cu") (free yes) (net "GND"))
 (via (at 162.7 99) (size 0.6) (drill 0.3) (layers "F.Cu" "B.Cu") (free yes) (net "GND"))
 (via (at 162 100.6) (size 0.6) (drill 0.3) (layers "F.Cu" "B.Cu") (free yes) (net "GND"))
 (via (at 163 106) (size 0.6) (drill 0.3) (layers "F.Cu" "B.Cu") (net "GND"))
 (via (at 158.9 96.9) (size 0.6) (drill 0.3) (layers "F.Cu" "B.Cu") (free yes) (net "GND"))
 (segment (start 162 104.51) (end 162.005 104.51) (width 0.2) (layer "F.Cu") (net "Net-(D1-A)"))
 (segment (start 162.005 104.51) (end 163 103.515) (width 0.2) (layer "F.Cu") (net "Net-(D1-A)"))
 (segment (start 159.75 103.25) (end 159.5 103.5) (width 0.2) (layer "F.Cu") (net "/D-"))
 (segment (start 159.75 102.4625) (end 159.75 103.25) (width 0.2) (layer "F.Cu") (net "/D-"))
 (via (at 159.5 103.5) (size 0.6) (drill 0.3) (layers "F.Cu" "B.Cu") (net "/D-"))
 (segment (start 160.25 102.4625) (end 160.25 103.25) (width 0.2) (layer "F.Cu") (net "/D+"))
 (segment (start 160.25 103.25) (end 160.5 103.5) (width 0.2) (layer "F.Cu") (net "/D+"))
 (via (at 160.5 103.5) (size 0.6) (drill 0.3) (layers "F.Cu" "B.Cu") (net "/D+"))
 (segment (start 160.75 102.901471) (end 161.338529 103.49) (width 0.2) (layer "F.Cu") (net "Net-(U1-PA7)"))
 (segment (start 161.338529 103.49) (end 162 103.49) (width 0.2) (layer "F.Cu") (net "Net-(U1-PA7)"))
 (segment (start 160.75 102.4625) (end 160.75 102.901471) (width 0.2) (layer "F.Cu") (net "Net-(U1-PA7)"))
 (segment (start 161.95 97.25) (end 161.95 98.462648) (width 0.2) (layer "F.Cu") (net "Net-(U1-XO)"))
 (segment (start 159.975 98.825) (end 159.75 99.05) (width 0.2) (layer "F.Cu") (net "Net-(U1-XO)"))
 (segment (start 161.587648 98.825) (end 159.975 98.825) (width 0.2) (layer "F.Cu") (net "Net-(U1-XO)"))
 (segment (start 161.65 96.95) (end 161.95 97.25) (width 0.2) (layer "F.Cu") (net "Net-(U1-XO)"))
 (segment (start 161.2 96.95) (end 161.65 96.95) (width 0.2) (layer "F.Cu") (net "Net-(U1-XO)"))
 (segment (start 159.75 99.05) (end 159.75 99.5375) (width 0.2) (layer "F.Cu") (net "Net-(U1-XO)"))
 (segment (start 161.95 98.462648) (end 161.587648 98.825) (width 0.2) (layer "F.Cu") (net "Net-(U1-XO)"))
 (segment (start 159.25 98.6) (end 159.25 99.5375) (width 0.2) (layer "F.Cu") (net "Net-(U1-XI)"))
 (segment (start 159.8 98.05) (end 159.25 98.6) (width 0.2) (layer "F.Cu") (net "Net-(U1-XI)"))
 (segment (start 156.29412 95.30588) (end 157.494363 96.506123) (width 0.5) (layer "F.Cu") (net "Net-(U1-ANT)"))
 (segment (start 155.90001 94.91177) (end 156.29412 95.30588) (width 0.2) (layer "F.Cu") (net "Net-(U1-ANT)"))
 (arc (start 158.667402 98.7) (mid 158.729303 99.116718) (end 158.75 99.5375) (width 0.2) (layer "F.Cu") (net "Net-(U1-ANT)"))
 (arc (start 157.494363 96.506123) (mid 158.243522 97.5161) (end 158.667402 98.7) (width 0.5) (layer "F.Cu") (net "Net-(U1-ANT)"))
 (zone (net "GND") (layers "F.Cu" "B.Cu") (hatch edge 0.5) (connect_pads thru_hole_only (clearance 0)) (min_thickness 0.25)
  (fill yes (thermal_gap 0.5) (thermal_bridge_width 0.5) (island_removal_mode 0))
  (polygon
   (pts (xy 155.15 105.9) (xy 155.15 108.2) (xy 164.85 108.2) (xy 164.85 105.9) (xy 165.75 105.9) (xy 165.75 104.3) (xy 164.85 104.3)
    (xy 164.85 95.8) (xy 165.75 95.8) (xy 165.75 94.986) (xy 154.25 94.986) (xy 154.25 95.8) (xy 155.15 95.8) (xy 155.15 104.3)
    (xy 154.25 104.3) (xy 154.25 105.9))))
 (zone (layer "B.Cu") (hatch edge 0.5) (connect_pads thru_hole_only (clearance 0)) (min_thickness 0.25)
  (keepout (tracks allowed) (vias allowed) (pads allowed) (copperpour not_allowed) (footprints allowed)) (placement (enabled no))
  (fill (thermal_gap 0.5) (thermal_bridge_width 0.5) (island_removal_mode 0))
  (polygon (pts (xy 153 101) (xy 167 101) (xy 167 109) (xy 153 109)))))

